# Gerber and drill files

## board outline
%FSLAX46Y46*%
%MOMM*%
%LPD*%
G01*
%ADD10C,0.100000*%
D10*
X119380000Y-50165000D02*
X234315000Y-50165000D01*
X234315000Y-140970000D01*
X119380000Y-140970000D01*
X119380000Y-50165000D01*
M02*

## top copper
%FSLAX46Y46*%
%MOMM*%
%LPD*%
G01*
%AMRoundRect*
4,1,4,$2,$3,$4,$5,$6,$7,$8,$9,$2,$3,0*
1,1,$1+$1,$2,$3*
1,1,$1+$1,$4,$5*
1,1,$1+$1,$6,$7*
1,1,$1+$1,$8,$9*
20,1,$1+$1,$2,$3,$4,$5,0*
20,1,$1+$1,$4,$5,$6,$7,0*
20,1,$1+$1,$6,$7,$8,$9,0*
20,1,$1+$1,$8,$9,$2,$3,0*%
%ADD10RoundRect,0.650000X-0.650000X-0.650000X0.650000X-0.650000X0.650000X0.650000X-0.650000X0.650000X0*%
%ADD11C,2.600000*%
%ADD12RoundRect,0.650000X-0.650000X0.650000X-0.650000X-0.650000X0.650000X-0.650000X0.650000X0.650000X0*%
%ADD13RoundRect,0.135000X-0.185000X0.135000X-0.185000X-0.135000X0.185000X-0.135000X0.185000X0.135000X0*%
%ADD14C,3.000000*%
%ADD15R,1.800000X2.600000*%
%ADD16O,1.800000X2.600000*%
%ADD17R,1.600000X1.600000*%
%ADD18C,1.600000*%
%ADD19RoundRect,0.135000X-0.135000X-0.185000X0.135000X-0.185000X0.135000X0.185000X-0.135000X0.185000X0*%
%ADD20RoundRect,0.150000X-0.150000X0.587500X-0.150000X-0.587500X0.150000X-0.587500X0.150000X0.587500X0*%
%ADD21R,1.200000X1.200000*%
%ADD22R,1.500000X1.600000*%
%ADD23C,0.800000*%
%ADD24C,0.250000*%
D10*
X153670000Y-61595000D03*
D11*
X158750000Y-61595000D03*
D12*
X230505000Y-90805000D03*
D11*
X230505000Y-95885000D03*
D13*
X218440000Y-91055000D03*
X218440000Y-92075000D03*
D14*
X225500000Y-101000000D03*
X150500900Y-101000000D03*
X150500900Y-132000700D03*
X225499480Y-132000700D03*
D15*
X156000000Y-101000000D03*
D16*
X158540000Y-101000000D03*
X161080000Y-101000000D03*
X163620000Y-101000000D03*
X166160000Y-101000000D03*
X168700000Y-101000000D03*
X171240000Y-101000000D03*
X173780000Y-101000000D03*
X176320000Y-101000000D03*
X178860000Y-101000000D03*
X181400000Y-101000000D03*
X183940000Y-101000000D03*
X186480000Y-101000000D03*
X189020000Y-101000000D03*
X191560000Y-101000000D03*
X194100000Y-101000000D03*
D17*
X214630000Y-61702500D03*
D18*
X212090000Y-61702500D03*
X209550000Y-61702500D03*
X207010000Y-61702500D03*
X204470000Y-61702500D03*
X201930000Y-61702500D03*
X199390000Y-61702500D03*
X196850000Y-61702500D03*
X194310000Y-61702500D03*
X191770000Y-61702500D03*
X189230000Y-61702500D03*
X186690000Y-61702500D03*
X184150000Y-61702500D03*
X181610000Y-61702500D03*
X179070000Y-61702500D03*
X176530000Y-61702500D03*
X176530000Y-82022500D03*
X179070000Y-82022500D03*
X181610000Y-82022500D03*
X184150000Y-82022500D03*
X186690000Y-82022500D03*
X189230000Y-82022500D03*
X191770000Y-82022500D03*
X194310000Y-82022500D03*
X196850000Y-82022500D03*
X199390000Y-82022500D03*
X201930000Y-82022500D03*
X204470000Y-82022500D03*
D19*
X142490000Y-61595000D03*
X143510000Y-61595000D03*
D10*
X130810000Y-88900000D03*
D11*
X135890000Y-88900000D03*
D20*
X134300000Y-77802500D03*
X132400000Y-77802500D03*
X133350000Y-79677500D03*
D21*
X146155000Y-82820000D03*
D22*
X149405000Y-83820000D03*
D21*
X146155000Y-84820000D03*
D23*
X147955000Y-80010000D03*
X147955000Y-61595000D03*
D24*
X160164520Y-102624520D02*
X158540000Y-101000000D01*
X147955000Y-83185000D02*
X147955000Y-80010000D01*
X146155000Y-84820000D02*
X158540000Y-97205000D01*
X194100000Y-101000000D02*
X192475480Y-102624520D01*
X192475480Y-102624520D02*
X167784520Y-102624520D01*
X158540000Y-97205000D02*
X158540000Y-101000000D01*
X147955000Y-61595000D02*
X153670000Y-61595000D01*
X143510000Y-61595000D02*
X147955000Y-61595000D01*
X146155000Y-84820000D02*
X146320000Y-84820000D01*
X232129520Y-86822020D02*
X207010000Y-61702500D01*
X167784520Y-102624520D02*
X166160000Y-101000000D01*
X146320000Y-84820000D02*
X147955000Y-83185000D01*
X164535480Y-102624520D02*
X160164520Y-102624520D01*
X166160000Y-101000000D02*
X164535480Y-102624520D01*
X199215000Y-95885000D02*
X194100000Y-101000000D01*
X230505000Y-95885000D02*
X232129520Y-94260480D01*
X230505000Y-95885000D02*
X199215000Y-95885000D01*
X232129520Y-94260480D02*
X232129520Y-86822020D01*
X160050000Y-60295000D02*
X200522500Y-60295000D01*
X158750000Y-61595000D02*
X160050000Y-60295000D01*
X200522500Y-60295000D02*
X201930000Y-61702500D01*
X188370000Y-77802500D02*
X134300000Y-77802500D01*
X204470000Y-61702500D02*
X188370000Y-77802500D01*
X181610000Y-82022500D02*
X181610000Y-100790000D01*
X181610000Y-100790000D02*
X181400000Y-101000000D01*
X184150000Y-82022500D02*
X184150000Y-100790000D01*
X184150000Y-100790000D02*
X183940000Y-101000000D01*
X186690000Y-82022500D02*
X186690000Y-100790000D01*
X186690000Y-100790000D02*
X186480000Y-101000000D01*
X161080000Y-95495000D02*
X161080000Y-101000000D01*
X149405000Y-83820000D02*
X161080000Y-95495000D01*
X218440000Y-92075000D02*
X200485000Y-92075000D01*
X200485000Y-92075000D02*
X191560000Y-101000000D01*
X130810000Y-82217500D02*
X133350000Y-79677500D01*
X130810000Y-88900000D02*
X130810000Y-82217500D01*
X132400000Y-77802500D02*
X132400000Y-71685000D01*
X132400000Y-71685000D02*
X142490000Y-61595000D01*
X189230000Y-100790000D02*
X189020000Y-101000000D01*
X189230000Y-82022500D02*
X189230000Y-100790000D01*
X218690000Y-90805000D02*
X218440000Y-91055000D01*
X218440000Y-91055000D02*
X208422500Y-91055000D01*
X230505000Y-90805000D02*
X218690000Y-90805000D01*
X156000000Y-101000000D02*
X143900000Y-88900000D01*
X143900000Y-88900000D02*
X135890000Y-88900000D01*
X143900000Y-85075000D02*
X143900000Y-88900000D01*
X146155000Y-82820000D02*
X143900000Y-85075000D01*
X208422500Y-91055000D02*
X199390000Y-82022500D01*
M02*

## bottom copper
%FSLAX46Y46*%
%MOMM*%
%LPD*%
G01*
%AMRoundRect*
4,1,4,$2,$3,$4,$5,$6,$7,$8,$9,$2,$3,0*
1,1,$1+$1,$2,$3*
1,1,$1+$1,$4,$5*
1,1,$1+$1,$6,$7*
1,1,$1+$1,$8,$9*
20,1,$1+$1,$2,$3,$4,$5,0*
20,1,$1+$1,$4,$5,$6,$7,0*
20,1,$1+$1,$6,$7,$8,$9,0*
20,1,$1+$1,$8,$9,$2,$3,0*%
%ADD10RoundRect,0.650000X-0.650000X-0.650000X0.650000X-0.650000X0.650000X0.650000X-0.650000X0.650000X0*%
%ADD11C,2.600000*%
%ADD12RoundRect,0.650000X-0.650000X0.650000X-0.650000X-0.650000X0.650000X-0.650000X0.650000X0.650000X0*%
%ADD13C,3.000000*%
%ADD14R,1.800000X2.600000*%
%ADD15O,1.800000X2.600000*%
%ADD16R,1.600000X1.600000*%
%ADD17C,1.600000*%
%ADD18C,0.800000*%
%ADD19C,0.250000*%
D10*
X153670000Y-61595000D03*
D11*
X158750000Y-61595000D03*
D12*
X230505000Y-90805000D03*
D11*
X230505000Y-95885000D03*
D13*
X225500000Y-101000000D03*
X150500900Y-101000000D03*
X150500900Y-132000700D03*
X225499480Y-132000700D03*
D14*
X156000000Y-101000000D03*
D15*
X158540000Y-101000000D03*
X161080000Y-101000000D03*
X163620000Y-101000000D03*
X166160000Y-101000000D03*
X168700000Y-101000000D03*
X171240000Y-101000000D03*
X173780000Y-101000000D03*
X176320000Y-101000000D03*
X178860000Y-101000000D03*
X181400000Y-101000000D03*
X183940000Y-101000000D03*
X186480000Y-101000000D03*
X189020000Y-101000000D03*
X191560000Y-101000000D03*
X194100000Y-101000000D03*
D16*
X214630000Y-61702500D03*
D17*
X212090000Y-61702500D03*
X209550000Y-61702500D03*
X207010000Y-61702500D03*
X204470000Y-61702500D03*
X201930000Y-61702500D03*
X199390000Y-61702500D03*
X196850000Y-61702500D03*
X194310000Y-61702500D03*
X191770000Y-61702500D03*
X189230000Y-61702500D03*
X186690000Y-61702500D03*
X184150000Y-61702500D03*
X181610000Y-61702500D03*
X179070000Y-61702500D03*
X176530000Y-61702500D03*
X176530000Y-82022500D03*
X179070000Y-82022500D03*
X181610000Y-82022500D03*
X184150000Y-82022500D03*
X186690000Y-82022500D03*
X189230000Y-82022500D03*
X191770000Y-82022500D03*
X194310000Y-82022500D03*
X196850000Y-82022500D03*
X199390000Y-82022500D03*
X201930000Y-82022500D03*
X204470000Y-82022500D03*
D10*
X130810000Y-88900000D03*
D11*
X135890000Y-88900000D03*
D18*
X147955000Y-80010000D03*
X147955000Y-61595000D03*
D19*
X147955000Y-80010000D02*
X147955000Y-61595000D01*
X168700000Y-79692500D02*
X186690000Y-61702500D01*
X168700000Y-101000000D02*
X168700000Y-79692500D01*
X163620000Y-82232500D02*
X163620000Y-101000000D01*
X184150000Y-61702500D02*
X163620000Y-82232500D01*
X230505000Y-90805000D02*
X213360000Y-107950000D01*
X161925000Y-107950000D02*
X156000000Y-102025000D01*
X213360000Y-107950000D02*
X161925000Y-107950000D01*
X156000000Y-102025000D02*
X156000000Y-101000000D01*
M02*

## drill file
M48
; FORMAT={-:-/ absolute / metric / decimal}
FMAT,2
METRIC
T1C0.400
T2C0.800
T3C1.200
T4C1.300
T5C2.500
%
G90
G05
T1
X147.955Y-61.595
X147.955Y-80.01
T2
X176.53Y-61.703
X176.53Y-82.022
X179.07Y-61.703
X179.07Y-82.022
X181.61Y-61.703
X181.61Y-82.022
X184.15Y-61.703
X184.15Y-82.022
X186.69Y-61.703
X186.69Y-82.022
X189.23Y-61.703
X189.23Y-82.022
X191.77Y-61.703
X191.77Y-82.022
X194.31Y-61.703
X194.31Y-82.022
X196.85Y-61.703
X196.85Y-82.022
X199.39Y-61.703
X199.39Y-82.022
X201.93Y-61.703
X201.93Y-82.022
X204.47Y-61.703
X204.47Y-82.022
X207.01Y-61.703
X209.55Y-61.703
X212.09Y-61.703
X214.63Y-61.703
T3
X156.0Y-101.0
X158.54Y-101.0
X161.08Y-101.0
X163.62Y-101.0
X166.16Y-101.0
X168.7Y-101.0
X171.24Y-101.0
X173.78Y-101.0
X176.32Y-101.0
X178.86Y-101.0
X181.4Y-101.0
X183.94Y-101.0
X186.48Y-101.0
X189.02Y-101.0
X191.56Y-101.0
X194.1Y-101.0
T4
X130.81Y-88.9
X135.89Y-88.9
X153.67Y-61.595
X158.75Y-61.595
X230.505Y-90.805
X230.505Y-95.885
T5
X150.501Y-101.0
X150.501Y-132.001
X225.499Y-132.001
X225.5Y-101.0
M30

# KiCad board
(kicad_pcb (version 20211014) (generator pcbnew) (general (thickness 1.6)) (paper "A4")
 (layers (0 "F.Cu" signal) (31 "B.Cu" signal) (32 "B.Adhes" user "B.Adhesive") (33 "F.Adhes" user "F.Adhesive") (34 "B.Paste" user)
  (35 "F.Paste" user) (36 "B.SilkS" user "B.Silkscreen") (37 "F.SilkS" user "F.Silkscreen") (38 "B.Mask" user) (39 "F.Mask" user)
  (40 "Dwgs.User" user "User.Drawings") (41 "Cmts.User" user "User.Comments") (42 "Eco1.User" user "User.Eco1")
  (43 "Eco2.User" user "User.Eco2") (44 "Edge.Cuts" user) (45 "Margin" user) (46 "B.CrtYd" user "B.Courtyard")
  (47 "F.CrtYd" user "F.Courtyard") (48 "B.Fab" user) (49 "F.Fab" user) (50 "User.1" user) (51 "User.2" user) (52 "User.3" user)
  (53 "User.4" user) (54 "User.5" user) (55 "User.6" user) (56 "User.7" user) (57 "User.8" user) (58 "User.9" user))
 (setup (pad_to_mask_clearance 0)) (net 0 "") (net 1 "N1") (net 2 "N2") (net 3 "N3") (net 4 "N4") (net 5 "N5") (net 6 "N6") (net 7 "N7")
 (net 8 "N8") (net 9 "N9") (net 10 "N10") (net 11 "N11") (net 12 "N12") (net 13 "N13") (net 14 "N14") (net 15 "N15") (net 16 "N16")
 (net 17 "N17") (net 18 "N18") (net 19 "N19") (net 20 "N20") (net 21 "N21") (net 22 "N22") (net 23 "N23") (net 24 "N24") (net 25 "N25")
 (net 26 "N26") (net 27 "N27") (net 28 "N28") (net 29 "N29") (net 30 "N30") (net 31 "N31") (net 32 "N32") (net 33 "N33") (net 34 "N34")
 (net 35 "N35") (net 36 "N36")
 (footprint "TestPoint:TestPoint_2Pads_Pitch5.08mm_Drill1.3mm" (layer "F.Cu") (at 153.67 61.595)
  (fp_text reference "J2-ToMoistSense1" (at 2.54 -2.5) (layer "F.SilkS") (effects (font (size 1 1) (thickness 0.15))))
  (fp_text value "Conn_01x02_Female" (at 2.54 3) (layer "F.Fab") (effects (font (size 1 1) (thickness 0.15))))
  (pad "1" thru_hole roundrect (at 0 0) (size 2.6 2.6) (drill 1.3) (layers *.Cu *.Mask) (roundrect_rratio 0.25) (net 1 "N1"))
  (pad "2" thru_hole circle (at 5.08 0) (size 2.6 2.6) (drill 1.3) (layers *.Cu *.Mask) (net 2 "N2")))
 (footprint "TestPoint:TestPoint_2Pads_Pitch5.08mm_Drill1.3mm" (layer "F.Cu") (at 230.505 90.805 -90)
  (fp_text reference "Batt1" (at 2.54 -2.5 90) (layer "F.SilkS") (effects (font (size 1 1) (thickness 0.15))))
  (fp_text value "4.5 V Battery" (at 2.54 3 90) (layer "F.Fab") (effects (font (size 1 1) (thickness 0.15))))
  (pad "1" thru_hole roundrect (at 0 0 270) (size 2.6 2.6) (drill 1.3) (layers *.Cu *.Mask) (roundrect_rratio 0.25) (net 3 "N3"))
  (pad "2" thru_hole circle (at 5.08 0 270) (size 2.6 2.6) (drill 1.3) (layers *.Cu *.Mask) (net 1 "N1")))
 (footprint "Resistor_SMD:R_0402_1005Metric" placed (layer "F.Cu") (at 218.44 91.565 -90)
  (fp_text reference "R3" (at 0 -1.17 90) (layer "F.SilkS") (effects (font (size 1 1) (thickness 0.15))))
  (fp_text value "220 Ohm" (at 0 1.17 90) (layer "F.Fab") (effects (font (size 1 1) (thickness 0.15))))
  (pad "1" smd roundrect (at -0.51 0 270) (size 0.54 0.64) (layers "F.Cu" "F.Paste" "F.Mask") (roundrect_rratio 0.25) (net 3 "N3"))
  (pad "2" smd roundrect (at 0.51 0 270) (size 0.54 0.64) (layers "F.Cu" "F.Paste" "F.Mask") (roundrect_rratio 0.25) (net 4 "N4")))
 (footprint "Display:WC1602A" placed (layer "F.Cu") (at 156 101)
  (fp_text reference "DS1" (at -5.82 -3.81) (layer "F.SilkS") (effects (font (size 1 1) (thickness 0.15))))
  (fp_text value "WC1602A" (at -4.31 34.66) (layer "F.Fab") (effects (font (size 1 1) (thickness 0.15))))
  (pad "" thru_hole circle (at 69.5 0) (size 3 3) (drill 2.5) (layers *.Cu *.Mask))
  (pad "" thru_hole circle (at -5.4991 0) (size 3 3) (drill 2.5) (layers *.Cu *.Mask))
  (pad "" thru_hole circle (at -5.4991 31.0007) (size 3 3) (drill 2.5) (layers *.Cu *.Mask))
  (pad "" thru_hole circle (at 69.49948 31.0007) (size 3 3) (drill 2.5) (layers *.Cu *.Mask))
  (pad "1" thru_hole rect (at 0 0) (size 1.8 2.6) (drill 1.2) (layers *.Cu *.Mask) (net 3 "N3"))
  (pad "2" thru_hole oval (at 2.54 0) (size 1.8 2.6) (drill 1.2) (layers *.Cu *.Mask) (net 1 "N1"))
  (pad "3" thru_hole oval (at 5.08 0) (size 1.8 2.6) (drill 1.2) (layers *.Cu *.Mask) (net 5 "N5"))
  (pad "4" thru_hole oval (at 7.62 0) (size 1.8 2.6) (drill 1.2) (layers *.Cu *.Mask) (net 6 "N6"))
  (pad "5" thru_hole oval (at 10.16 0) (size 1.8 2.6) (drill 1.2) (layers *.Cu *.Mask) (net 1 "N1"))
  (pad "6" thru_hole oval (at 12.7 0) (size 1.8 2.6) (drill 1.2) (layers *.Cu *.Mask) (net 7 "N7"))
  (pad "7" thru_hole oval (at 15.24 0) (size 1.8 2.6) (drill 1.2) (layers *.Cu *.Mask) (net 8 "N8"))
  (pad "8" thru_hole oval (at 17.78 0) (size 1.8 2.6) (drill 1.2) (layers *.Cu *.Mask) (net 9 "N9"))
  (pad "9" thru_hole oval (at 20.32 0) (size 1.8 2.6) (drill 1.2) (layers *.Cu *.Mask) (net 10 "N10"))
  (pad "10" thru_hole oval (at 22.86 0) (size 1.8 2.6) (drill 1.2) (layers *.Cu *.Mask) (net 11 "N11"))
  (pad "11" thru_hole oval (at 25.4 0) (size 1.8 2.6) (drill 1.2) (layers *.Cu *.Mask) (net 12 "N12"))
  (pad "12" thru_hole oval (at 27.94 0) (size 1.8 2.6) (drill 1.2) (layers *.Cu *.Mask) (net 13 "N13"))
  (pad "13" thru_hole oval (at 30.48 0) (size 1.8 2.6) (drill 1.2) (layers *.Cu *.Mask) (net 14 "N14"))
  (pad "14" thru_hole oval (at 33.02 0) (size 1.8 2.6) (drill 1.2) (layers *.Cu *.Mask) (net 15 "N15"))
  (pad "15" thru_hole oval (at 35.56 0) (size 1.8 2.6) (drill 1.2) (layers *.Cu *.Mask) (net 4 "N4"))
  (pad "16" thru_hole oval (at 38.1 0) (size 1.8 2.6) (drill 1.2) (layers *.Cu *.Mask) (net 1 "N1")))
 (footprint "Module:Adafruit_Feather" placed (layer "F.Cu") (at 214.63 61.7025 -90)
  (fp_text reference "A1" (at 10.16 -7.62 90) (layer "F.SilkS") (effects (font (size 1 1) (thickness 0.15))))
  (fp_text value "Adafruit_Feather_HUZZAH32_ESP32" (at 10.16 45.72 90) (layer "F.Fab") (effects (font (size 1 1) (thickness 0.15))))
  (pad "1" thru_hole rect (at 0 0 90) (size 1.6 1.6) (drill 0.8) (layers *.Cu *.Mask) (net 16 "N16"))
  (pad "2" thru_hole circle (at 0 2.54 90) (size 1.6 1.6) (drill 0.8) (layers *.Cu *.Mask) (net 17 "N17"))
  (pad "3" thru_hole circle (at 0 5.08 90) (size 1.6 1.6) (drill 0.8) (layers *.Cu *.Mask) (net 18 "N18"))
  (pad "4" thru_hole circle (at 0 7.62 90) (size 1.6 1.6) (drill 0.8) (layers *.Cu *.Mask) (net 1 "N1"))
  (pad "5" thru_hole circle (at 0 10.16 90) (size 1.6 1.6) (drill 0.8) (layers *.Cu *.Mask) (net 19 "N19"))
  (pad "6" thru_hole circle (at 0 12.7 90) (size 1.6 1.6) (drill 0.8) (layers *.Cu *.Mask) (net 2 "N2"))
  (pad "7" thru_hole circle (at 0 15.24 90) (size 1.6 1.6) (drill 0.8) (layers *.Cu *.Mask) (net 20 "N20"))
  (pad "8" thru_hole circle (at 0 17.78 90) (size 1.6 1.6) (drill 0.8) (layers *.Cu *.Mask) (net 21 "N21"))
  (pad "9" thru_hole circle (at 0 20.32 90) (size 1.6 1.6) (drill 0.8) (layers *.Cu *.Mask) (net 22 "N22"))
  (pad "10" thru_hole circle (at 0 22.86 90) (size 1.6 1.6) (drill 0.8) (layers *.Cu *.Mask) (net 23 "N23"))
  (pad "11" thru_hole circle (at 0 25.4 90) (size 1.6 1.6) (drill 0.8) (layers *.Cu *.Mask) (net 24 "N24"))
  (pad "12" thru_hole circle (at 0 27.94 90) (size 1.6 1.6) (drill 0.8) (layers *.Cu *.Mask) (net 7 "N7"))
  (pad "13" thru_hole circle (at 0 30.48 90) (size 1.6 1.6) (drill 0.8) (layers *.Cu *.Mask) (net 6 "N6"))
  (pad "14" thru_hole circle (at 0 33.02 90) (size 1.6 1.6) (drill 0.8) (layers *.Cu *.Mask) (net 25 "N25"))
  (pad "15" thru_hole circle (at 0 35.56 90) (size 1.6 1.6) (drill 0.8) (layers *.Cu *.Mask) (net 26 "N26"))
  (pad "16" thru_hole circle (at 0 38.1 90) (size 1.6 1.6) (drill 0.8) (layers *.Cu *.Mask) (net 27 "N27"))
  (pad "17" thru_hole circle (at 20.32 38.1 90) (size 1.6 1.6) (drill 0.8) (layers *.Cu *.Mask) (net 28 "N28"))
  (pad "18" thru_hole circle (at 20.32 35.56 90) (size 1.6 1.6) (drill 0.8) (layers *.Cu *.Mask) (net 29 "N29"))
  (pad "19" thru_hole circle (at 20.32 33.02 90) (size 1.6 1.6) (drill 0.8) (layers *.Cu *.Mask) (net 12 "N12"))
  (pad "20" thru_hole circle (at 20.32 30.48 90) (size 1.6 1.6) (drill 0.8) (layers *.Cu *.Mask) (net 13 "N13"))
  (pad "21" thru_hole circle (at 20.32 27.94 90) (size 1.6 1.6) (drill 0.8) (layers *.Cu *.Mask) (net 14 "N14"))
  (pad "22" thru_hole circle (at 20.32 25.4 90) (size 1.6 1.6) (drill 0.8) (layers *.Cu *.Mask) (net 15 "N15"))
  (pad "23" thru_hole circle (at 20.32 22.86 90) (size 1.6 1.6) (drill 0.8) (layers *.Cu *.Mask) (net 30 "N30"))
  (pad "24" thru_hole circle (at 20.32 20.32 90) (size 1.6 1.6) (drill 0.8) (layers *.Cu *.Mask) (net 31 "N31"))
  (pad "25" thru_hole circle (at 20.32 17.78 90) (size 1.6 1.6) (drill 0.8) (layers *.Cu *.Mask) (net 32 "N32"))
  (pad "26" thru_hole circle (at 20.32 15.24 90) (size 1.6 1.6) (drill 0.8) (layers *.Cu *.Mask) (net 3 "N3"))
  (pad "27" thru_hole circle (at 20.32 12.7 90) (size 1.6 1.6) (drill 0.8) (layers *.Cu *.Mask) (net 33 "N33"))
  (pad "28" thru_hole circle (at 20.32 10.16 90) (size 1.6 1.6) (drill 0.8) (layers *.Cu *.Mask) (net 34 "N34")))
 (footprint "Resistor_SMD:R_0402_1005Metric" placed (layer "F.Cu") (at 143 61.595)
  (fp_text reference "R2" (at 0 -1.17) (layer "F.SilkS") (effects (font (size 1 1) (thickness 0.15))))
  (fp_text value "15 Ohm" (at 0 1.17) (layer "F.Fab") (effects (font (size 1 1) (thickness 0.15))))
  (pad "1" smd roundrect (at -0.51 0) (size 0.54 0.64) (layers "F.Cu" "F.Paste" "F.Mask") (roundrect_rratio 0.25) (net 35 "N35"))
  (pad "2" smd roundrect (at 0.51 0) (size 0.54 0.64) (layers "F.Cu" "F.Paste" "F.Mask") (roundrect_rratio 0.25) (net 1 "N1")))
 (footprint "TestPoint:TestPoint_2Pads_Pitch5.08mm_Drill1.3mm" (layer "F.Cu") (at 130.81 88.9)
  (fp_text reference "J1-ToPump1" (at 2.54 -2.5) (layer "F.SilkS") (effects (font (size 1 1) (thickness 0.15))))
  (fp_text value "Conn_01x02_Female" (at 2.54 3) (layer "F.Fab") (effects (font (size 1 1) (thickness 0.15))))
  (pad "1" thru_hole roundrect (at 0 0) (size 2.6 2.6) (drill 1.3) (layers *.Cu *.Mask) (roundrect_rratio 0.25) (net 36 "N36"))
  (pad "2" thru_hole circle (at 5.08 0) (size 2.6 2.6) (drill 1.3) (layers *.Cu *.Mask) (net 3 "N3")))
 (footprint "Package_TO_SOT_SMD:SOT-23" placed (layer "F.Cu") (at 133.35 78.74 -90)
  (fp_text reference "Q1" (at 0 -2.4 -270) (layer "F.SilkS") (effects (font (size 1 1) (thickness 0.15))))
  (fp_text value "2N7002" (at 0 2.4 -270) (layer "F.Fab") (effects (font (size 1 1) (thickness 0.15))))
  (pad "1" smd roundrect (at -0.9375 -0.95 270) (size 1.475 0.6) (layers "F.Cu" "F.Paste" "F.Mask") (roundrect_rratio 0.25) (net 19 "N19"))
  (pad "2" smd roundrect (at -0.9375 0.95 270) (size 1.475 0.6) (layers "F.Cu" "F.Paste" "F.Mask") (roundrect_rratio 0.25) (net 35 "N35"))
  (pad "3" smd roundrect (at 0.9375 0 270) (size 1.475 0.6) (layers "F.Cu" "F.Paste" "F.Mask") (roundrect_rratio 0.25) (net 36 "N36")))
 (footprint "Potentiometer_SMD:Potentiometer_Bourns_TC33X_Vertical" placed (layer "F.Cu") (at 147.955 83.82)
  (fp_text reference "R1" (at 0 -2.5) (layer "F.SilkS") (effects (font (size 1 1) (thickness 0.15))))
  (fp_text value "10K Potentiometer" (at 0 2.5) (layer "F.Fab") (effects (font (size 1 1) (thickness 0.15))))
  (pad "1" smd rect (at -1.8 -1) (size 1.2 1.2) (layers "F.Cu" "F.Paste" "F.Mask") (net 3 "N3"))
  (pad "2" smd rect (at 1.45 0) (size 1.5 1.6) (layers "F.Cu" "F.Paste" "F.Mask") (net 5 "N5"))
  (pad "3" smd rect (at -1.8 1) (size 1.2 1.2) (layers "F.Cu" "F.Paste" "F.Mask") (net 1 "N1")))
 (gr_rect (start 119.38 140.97) (end 234.315 50.165) (layer "Edge.Cuts") (width 0.1) (fill none))
 (segment (start 160.16452 102.62452) (end 158.54 101) (width 0.25) (layer "F.Cu") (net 1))
 (segment (start 147.955 83.185) (end 147.955 80.01) (width 0.25) (layer "F.Cu") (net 1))
 (segment (start 146.155 84.82) (end 158.54 97.205) (width 0.25) (layer "F.Cu") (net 1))
 (segment (start 194.1 101) (end 192.47548 102.62452) (width 0.25) (layer "F.Cu") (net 1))
 (segment (start 192.47548 102.62452) (end 167.78452 102.62452) (width 0.25) (layer "F.Cu") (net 1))
 (segment (start 158.54 97.205) (end 158.54 101) (width 0.25) (layer "F.Cu") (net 1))
 (segment (start 147.955 61.595) (end 153.67 61.595) (width 0.25) (layer "F.Cu") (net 1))
 (segment (start 143.51 61.595) (end 147.955 61.595) (width 0.25) (layer "F.Cu") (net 1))
 (segment (start 146.155 84.82) (end 146.32 84.82) (width 0.25) (layer "F.Cu") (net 1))
 (segment (start 232.12952 86.82202) (end 207.01 61.7025) (width 0.25) (layer "F.Cu") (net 1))
 (segment (start 167.78452 102.62452) (end 166.16 101) (width 0.25) (layer "F.Cu") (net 1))
 (segment (start 146.32 84.82) (end 147.955 83.185) (width 0.25) (layer "F.Cu") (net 1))
 (segment (start 164.53548 102.62452) (end 160.16452 102.62452) (width 0.25) (layer "F.Cu") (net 1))
 (segment (start 166.16 101) (end 164.53548 102.62452) (width 0.25) (layer "F.Cu") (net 1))
 (segment (start 199.215 95.885) (end 194.1 101) (width 0.25) (layer "F.Cu") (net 1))
 (segment (start 230.505 95.885) (end 232.12952 94.26048) (width 0.25) (layer "F.Cu") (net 1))
 (segment (start 230.505 95.885) (end 199.215 95.885) (width 0.25) (layer "F.Cu") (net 1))
 (segment (start 232.12952 94.26048) (end 232.12952 86.82202) (width 0.25) (layer "F.Cu") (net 1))
 (via (at 147.955 80.01) (size 0.8) (drill 0.4) (layers "F.Cu" "B.Cu") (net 1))
 (via (at 147.955 61.595) (size 0.8) (drill 0.4) (layers "F.Cu" "B.Cu") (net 1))
 (segment (start 147.955 80.01) (end 147.955 61.595) (width 0.25) (layer "B.Cu") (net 1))
 (segment (start 160.05 60.295) (end 200.5225 60.295) (width 0.25) (layer "F.Cu") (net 2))
 (segment (start 158.75 61.595) (end 160.05 60.295) (width 0.25) (layer "F.Cu") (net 2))
 (segment (start 200.5225 60.295) (end 201.93 61.7025) (width 0.25) (layer "F.Cu") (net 2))
 (segment (start 188.37 77.8025) (end 134.3 77.8025) (width 0.25) (layer "F.Cu") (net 19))
 (segment (start 204.47 61.7025) (end 188.37 77.8025) (width 0.25) (layer "F.Cu") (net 19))
 (segment (start 181.61 82.0225) (end 181.61 100.79) (width 0.25) (layer "F.Cu") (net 12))
 (segment (start 181.61 100.79) (end 181.4 101) (width 0.25) (layer "F.Cu") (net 12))
 (segment (start 184.15 82.0225) (end 184.15 100.79) (width 0.25) (layer "F.Cu") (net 13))
 (segment (start 184.15 100.79) (end 183.94 101) (width 0.25) (layer "F.Cu") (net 13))
 (segment (start 186.69 82.0225) (end 186.69 100.79) (width 0.25) (layer "F.Cu") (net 14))
 (segment (start 186.69 100.79) (end 186.48 101) (width 0.25) (layer "F.Cu") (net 14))
 (segment (start 161.08 95.495) (end 161.08 101) (width 0.25) (layer "F.Cu") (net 5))
 (segment (start 149.405 83.82) (end 161.08 95.495) (width 0.25) (layer "F.Cu") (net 5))
 (segment (start 218.44 92.075) (end 200.485 92.075) (width 0.25) (layer "F.Cu") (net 4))
 (segment (start 200.485 92.075) (end 191.56 101) (width 0.25) (layer "F.Cu") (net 4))
 (segment (start 130.81 82.2175) (end 133.35 79.6775) (width 0.25) (layer "F.Cu") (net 36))
 (segment (start 130.81 88.9) (end 130.81 82.2175) (width 0.25) (layer "F.Cu") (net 36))
 (segment (start 132.4 77.8025) (end 132.4 71.685) (width 0.25) (layer "F.Cu") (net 35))
 (segment (start 132.4 71.685) (end 142.49 61.595) (width 0.25) (layer "F.Cu") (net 35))
 (segment (start 168.7 79.6925) (end 186.69 61.7025) (width 0.25) (layer "B.Cu") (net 7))
 (segment (start 168.7 101) (end 168.7 79.6925) (width 0.25) (layer "B.Cu") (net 7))
 (segment (start 163.62 82.2325) (end 163.62 101) (width 0.25) (layer "B.Cu") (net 6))
 (segment (start 184.15 61.7025) (end 163.62 82.2325) (width 0.25) (layer "B.Cu") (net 6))
 (segment (start 189.23 100.79) (end 189.02 101) (width 0.25) (layer "F.Cu") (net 15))
 (segment (start 189.23 82.0225) (end 189.23 100.79) (width 0.25) (layer "F.Cu") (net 15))
 (segment (start 218.69 90.805) (end 218.44 91.055) (width 0.25) (layer "F.Cu") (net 3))
 (segment (start 218.44 91.055) (end 208.4225 91.055) (width 0.25) (layer "F.Cu") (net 3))
 (segment (start 230.505 90.805) (end 218.69 90.805) (width 0.25) (layer "F.Cu") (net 3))
 (segment (start 156 101) (end 143.9 88.9) (width 0.25) (layer "F.Cu") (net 3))
 (segment (start 143.9 88.9) (end 135.89 88.9) (width 0.25) (layer "F.Cu") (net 3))
 (segment (start 143.9 85.075) (end 143.9 88.9) (width 0.25) (layer "F.Cu") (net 3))
 (segment (start 146.155 82.82) (end 143.9 85.075) (width 0.25) (layer "F.Cu") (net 3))
 (segment (start 208.4225 91.055) (end 199.39 82.0225) (width 0.25) (layer "F.Cu") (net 3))
 (segment (start 230.505 90.805) (end 213.36 107.95) (width 0.25) (layer "B.Cu") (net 3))
 (segment (start 161.925 107.95) (end 156 102.025) (width 0.25) (layer "B.Cu") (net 3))
 (segment (start 213.36 107.95) (end 161.925 107.95) (width 0.25) (layer "B.Cu") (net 3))
 (segment (start 156 102.025) (end 156 101) (width 0.25) (layer "B.Cu") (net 3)))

